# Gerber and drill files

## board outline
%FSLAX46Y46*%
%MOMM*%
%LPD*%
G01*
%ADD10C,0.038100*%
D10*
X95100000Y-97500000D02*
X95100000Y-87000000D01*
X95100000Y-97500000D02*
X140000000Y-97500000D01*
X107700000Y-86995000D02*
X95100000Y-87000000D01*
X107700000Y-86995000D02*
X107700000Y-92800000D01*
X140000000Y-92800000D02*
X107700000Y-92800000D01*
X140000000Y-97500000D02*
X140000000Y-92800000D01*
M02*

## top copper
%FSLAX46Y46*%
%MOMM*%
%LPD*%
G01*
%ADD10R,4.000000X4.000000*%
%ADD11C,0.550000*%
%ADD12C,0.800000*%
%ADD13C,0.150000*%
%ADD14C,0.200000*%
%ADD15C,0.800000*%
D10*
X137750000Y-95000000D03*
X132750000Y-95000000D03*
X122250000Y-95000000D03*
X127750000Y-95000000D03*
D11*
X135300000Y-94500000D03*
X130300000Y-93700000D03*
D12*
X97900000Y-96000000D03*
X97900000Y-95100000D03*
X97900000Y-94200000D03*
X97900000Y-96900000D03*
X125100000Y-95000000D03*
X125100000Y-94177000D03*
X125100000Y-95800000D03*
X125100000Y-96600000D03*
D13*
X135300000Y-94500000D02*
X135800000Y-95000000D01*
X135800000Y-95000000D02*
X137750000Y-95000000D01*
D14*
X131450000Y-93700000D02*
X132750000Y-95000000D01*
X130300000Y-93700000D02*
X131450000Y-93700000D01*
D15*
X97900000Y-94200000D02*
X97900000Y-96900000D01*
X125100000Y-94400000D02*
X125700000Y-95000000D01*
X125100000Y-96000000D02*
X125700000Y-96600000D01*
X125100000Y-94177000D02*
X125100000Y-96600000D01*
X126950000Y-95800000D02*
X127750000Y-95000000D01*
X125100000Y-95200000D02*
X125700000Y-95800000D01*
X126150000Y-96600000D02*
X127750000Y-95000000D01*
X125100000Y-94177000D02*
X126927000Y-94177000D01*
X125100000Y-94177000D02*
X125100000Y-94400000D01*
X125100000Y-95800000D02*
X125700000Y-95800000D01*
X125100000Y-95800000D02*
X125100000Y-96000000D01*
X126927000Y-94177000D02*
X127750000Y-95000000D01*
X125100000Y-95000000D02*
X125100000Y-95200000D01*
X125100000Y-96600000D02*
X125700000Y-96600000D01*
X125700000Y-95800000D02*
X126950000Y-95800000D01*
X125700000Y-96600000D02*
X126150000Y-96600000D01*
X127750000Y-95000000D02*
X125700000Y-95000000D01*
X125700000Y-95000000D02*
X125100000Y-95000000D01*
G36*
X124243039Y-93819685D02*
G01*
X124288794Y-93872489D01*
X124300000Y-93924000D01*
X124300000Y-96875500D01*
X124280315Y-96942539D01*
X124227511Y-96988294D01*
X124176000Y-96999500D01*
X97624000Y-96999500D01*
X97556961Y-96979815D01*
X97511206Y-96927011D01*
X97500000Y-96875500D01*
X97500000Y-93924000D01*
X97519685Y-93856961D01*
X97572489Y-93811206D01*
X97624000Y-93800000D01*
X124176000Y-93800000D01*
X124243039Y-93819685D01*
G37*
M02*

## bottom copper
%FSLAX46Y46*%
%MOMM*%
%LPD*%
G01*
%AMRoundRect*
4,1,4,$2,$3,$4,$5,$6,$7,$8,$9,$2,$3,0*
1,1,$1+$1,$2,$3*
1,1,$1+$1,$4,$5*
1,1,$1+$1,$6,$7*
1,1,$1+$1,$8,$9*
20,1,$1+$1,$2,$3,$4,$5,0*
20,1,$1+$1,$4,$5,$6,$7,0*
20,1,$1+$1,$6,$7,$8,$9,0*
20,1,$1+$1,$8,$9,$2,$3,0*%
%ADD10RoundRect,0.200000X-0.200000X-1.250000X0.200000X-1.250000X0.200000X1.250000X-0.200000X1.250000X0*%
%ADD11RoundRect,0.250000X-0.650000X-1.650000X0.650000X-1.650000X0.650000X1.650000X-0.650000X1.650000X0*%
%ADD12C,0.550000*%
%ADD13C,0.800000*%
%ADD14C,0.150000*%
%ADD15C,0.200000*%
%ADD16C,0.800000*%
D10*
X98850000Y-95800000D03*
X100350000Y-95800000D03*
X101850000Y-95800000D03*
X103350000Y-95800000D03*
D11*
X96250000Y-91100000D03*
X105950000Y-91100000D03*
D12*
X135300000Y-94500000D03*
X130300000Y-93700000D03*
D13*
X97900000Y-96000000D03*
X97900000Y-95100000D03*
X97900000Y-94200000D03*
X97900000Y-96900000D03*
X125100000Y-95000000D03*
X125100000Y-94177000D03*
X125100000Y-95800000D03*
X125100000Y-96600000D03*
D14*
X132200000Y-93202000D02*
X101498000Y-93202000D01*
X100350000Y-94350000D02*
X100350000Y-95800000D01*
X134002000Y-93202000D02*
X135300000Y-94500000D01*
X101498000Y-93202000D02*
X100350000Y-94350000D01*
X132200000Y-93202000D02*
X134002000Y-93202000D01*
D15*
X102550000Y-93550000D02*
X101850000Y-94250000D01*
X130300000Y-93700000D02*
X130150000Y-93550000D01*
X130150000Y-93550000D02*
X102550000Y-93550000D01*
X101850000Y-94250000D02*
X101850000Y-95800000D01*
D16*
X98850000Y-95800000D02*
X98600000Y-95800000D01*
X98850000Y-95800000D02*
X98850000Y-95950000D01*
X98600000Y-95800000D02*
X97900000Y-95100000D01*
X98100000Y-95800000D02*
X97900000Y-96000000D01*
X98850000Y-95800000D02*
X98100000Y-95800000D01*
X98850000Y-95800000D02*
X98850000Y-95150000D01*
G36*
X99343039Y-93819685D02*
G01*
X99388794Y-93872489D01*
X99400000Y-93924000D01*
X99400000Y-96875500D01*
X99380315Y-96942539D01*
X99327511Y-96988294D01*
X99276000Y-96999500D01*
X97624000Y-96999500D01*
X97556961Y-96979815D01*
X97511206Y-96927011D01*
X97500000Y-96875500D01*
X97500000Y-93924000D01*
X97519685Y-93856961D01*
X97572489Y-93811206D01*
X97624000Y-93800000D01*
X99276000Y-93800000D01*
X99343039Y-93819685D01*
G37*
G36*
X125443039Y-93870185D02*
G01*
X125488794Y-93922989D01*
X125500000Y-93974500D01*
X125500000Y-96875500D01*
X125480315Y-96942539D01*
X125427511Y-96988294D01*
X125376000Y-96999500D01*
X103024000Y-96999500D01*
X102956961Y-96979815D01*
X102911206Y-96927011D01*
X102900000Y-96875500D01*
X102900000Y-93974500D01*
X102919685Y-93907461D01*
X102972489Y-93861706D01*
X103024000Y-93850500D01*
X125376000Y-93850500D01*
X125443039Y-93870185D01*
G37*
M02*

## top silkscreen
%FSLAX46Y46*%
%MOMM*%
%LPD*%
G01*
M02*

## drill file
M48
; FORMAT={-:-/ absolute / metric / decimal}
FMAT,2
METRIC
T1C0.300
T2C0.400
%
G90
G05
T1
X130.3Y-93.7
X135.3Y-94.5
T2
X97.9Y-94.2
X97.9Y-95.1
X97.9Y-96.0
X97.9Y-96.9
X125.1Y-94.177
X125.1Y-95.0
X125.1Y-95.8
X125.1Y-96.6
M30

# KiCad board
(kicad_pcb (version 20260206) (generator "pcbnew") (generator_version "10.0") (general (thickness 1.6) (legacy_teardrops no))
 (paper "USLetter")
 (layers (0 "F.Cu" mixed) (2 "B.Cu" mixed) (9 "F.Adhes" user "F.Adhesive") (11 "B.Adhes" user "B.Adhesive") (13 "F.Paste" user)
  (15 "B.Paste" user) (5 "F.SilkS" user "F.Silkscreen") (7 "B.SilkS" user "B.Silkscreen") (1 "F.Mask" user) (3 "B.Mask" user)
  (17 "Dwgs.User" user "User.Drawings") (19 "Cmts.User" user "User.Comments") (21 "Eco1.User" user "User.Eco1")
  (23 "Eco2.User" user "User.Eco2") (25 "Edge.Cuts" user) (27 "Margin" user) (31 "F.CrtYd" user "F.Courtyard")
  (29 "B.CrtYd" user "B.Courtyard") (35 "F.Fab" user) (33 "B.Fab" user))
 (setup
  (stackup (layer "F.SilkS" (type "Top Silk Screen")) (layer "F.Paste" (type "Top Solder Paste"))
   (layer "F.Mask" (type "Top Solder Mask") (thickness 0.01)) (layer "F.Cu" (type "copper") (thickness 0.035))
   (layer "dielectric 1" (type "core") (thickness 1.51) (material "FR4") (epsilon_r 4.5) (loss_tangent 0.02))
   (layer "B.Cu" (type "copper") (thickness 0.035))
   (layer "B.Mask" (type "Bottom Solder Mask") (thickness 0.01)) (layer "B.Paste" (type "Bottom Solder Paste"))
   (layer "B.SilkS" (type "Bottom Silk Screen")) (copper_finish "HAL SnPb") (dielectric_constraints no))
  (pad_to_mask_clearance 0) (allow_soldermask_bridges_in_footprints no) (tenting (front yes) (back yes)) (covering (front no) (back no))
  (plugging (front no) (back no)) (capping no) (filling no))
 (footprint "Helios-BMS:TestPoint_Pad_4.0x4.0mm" (layer "F.Cu") (at 137.75 95)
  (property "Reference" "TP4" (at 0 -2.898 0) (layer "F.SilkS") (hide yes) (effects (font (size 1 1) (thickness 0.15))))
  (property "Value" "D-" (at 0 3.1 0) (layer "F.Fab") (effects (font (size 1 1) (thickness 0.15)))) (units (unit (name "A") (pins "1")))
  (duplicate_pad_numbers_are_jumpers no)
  (pad "1" smd rect (at 0 0) (size 4 4) (layers "F.Cu" "F.Mask") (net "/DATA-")))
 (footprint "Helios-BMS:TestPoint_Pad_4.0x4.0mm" (layer "F.Cu") (at 133.25 95)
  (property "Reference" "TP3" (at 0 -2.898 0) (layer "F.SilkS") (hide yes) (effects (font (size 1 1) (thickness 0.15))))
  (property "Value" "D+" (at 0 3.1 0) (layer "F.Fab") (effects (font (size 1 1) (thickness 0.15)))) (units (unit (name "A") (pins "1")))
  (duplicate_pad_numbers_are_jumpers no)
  (pad "1" smd rect (at -0.5 0) (size 4 4) (layers "F.Cu" "F.Mask") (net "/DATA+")))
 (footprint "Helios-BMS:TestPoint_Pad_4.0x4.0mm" (layer "F.Cu") (at 131 95)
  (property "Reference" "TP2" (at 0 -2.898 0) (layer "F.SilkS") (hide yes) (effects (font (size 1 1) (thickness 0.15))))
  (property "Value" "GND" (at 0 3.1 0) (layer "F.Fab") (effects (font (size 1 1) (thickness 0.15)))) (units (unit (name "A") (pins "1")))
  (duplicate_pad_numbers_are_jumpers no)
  (pad "1" smd rect (at -8.75 0) (size 4 4) (layers "F.Cu" "F.Mask") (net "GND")))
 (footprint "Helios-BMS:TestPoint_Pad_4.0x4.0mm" (layer "F.Cu") (at 122.75 95)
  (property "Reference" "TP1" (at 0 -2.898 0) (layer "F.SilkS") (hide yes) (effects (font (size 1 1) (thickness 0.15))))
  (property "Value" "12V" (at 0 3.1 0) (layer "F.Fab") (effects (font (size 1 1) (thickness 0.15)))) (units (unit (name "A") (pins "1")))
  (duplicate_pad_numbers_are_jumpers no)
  (pad "1" smd rect (at 5 0) (size 4 4) (layers "F.Cu" "F.Mask") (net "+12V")))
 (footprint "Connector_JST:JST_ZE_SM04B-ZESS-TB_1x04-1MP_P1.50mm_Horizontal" (layer "B.Cu") (at 101.1 93.225)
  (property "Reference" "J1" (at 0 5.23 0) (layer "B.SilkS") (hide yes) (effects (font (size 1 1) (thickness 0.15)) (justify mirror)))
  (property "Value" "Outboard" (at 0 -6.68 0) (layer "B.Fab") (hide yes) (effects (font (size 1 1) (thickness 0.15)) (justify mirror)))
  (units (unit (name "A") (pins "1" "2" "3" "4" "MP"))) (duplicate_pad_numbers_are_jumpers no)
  (pad "1" smd roundrect (at -2.25 2.575) (size 0.8 2.9) (layers "B.Cu" "B.Mask" "B.Paste") (roundrect_rratio 0.25) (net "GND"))
  (pad "2" smd roundrect (at -0.75 2.575) (size 0.8 2.9) (layers "B.Cu" "B.Mask" "B.Paste") (roundrect_rratio 0.25) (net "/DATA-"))
  (pad "3" smd roundrect (at 0.75 2.575) (size 0.8 2.9) (layers "B.Cu" "B.Mask" "B.Paste") (roundrect_rratio 0.25) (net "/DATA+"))
  (pad "4" smd roundrect (at 2.25 2.575) (size 0.8 2.9) (layers "B.Cu" "B.Mask" "B.Paste") (roundrect_rratio 0.25) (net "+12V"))
  (pad "MP" smd roundrect (at -4.85 -2.125) (size 1.8 3.8) (layers "B.Cu" "B.Mask" "B.Paste") (roundrect_rratio 0.138889)
   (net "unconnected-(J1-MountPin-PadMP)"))
  (pad "MP" smd roundrect (at 4.85 -2.125) (size 1.8 3.8) (layers "B.Cu" "B.Mask" "B.Paste") (roundrect_rratio 0.138889)
   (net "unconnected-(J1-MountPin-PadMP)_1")))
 (gr_line (start 95.1 97.5) (end 95.1 87) (stroke (width 0.0381) (type default)) (layer "Edge.Cuts"))
 (gr_line (start 95.1 97.5) (end 140 97.5) (stroke (width 0.0381) (type solid)) (layer "Edge.Cuts"))
 (gr_line (start 107.7 86.995) (end 95.1 87) (stroke (width 0.0381) (type default)) (layer "Edge.Cuts"))
 (gr_line (start 107.7 86.995) (end 107.7 92.8) (stroke (width 0.0381) (type default)) (layer "Edge.Cuts"))
 (gr_line (start 140 92.8) (end 107.7 92.8) (stroke (width 0.0381) (type default)) (layer "Edge.Cuts"))
 (gr_line (start 140 97.5) (end 140 92.8) (stroke (width 0.0381) (type solid)) (layer "Edge.Cuts"))
 (segment (start 135.3 94.5) (end 135.8 95) (width 0.15) (layer "F.Cu") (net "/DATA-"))
 (segment (start 135.8 95) (end 137.75 95) (width 0.15) (layer "F.Cu") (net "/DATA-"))
 (via (at 135.3 94.5) (size 0.55) (drill 0.3) (layers "F.Cu" "B.Cu") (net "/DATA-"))
 (segment (start 132.2 93.202) (end 101.498 93.202) (width 0.15) (layer "B.Cu") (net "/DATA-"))
 (segment (start 100.35 94.35) (end 100.35 95.8) (width 0.15) (layer "B.Cu") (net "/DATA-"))
 (segment (start 134.002 93.202) (end 135.3 94.5) (width 0.15) (layer "B.Cu") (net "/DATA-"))
 (segment (start 101.498 93.202) (end 100.35 94.35) (width 0.15) (layer "B.Cu") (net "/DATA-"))
 (segment (start 132.2 93.202) (end 134.002 93.202) (width 0.15) (layer "B.Cu") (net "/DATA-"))
 (segment (start 131.45 93.7) (end 132.75 95) (width 0.2) (layer "F.Cu") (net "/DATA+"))
 (segment (start 130.3 93.7) (end 131.45 93.7) (width 0.2) (layer "F.Cu") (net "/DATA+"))
 (via (at 130.3 93.7) (size 0.55) (drill 0.3) (layers "F.Cu" "B.Cu") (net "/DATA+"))
 (segment (start 102.55 93.55) (end 101.85 94.25) (width 0.2) (layer "B.Cu") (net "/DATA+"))
 (segment (start 130.3 93.7) (end 130.15 93.55) (width 0.2) (layer "B.Cu") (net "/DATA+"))
 (segment (start 130.15 93.55) (end 102.55 93.55) (width 0.2) (layer "B.Cu") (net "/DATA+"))
 (segment (start 101.85 94.25) (end 101.85 95.8) (width 0.2) (layer "B.Cu") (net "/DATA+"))
 (segment (start 97.9 94.2) (end 97.9 96.9) (width 0.8) (layer "F.Cu") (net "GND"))
 (via (at 97.9 96) (size 0.8) (drill 0.4) (layers "F.Cu" "B.Cu") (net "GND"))
 (via (at 97.9 95.1) (size 0.8) (drill 0.4) (layers "F.Cu" "B.Cu") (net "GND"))
 (via (at 97.9 94.2) (size 0.8) (drill 0.4) (layers "F.Cu" "B.Cu") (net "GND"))
 (via (at 97.9 96.9) (size 0.8) (drill 0.4) (layers "F.Cu" "B.Cu") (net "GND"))
 (segment (start 98.85 95.8) (end 98.6 95.8) (width 0.8) (layer "B.Cu") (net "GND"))
 (segment (start 98.85 95.8) (end 98.85 95.95) (width 0.8) (layer "B.Cu") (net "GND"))
 (segment (start 98.6 95.8) (end 97.9 95.1) (width 0.8) (layer "B.Cu") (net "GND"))
 (segment (start 98.1 95.8) (end 97.9 96) (width 0.8) (layer "B.Cu") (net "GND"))
 (segment (start 98.85 95.8) (end 98.1 95.8) (width 0.8) (layer "B.Cu") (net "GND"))
 (segment (start 98.85 95.8) (end 98.85 95.15) (width 0.8) (layer "B.Cu") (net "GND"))
 (segment (start 125.1 94.4) (end 125.7 95) (width 0.8) (layer "F.Cu") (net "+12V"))
 (segment (start 125.1 96) (end 125.7 96.6) (width 0.8) (layer "F.Cu") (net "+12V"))
 (segment (start 125.1 94.177) (end 125.1 96.6) (width 0.8) (layer "F.Cu") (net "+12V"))
 (segment (start 126.95 95.8) (end 127.75 95) (width 0.8) (layer "F.Cu") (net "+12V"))
 (segment (start 125.1 95.2) (end 125.7 95.8) (width 0.8) (layer "F.Cu") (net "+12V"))
 (segment (start 126.15 96.6) (end 127.75 95) (width 0.8) (layer "F.Cu") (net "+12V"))
 (segment (start 125.1 94.177) (end 126.927 94.177) (width 0.8) (layer "F.Cu") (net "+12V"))
 (segment (start 125.1 94.177) (end 125.1 94.4) (width 0.8) (layer "F.Cu") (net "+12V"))
 (segment (start 125.1 95.8) (end 125.7 95.8) (width 0.8) (layer "F.Cu") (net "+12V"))
 (segment (start 125.1 95.8) (end 125.1 96) (width 0.8) (layer "F.Cu") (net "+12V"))
 (segment (start 126.927 94.177) (end 127.75 95) (width 0.8) (layer "F.Cu") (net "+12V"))
 (segment (start 125.1 95) (end 125.1 95.2) (width 0.8) (layer "F.Cu") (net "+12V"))
 (segment (start 125.1 96.6) (end 125.7 96.6) (width 0.8) (layer "F.Cu") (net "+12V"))
 (segment (start 125.7 95.8) (end 126.95 95.8) (width 0.8) (layer "F.Cu") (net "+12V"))
 (segment (start 125.7 96.6) (end 126.15 96.6) (width 0.8) (layer "F.Cu") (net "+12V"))
 (segment (start 127.75 95) (end 125.7 95) (width 0.8) (layer "F.Cu") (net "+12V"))
 (segment (start 125.7 95) (end 125.1 95) (width 0.8) (layer "F.Cu") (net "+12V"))
 (via (at 125.1 95) (size 0.8) (drill 0.4) (layers "F.Cu" "B.Cu") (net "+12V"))
 (via (at 125.1 94.177) (size 0.8) (drill 0.4) (layers "F.Cu" "B.Cu") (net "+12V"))
 (via (at 125.1 95.8) (size 0.8) (drill 0.4) (layers "F.Cu" "B.Cu") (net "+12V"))
 (via (at 125.1 96.6) (size 0.8) (drill 0.4) (layers "F.Cu" "B.Cu") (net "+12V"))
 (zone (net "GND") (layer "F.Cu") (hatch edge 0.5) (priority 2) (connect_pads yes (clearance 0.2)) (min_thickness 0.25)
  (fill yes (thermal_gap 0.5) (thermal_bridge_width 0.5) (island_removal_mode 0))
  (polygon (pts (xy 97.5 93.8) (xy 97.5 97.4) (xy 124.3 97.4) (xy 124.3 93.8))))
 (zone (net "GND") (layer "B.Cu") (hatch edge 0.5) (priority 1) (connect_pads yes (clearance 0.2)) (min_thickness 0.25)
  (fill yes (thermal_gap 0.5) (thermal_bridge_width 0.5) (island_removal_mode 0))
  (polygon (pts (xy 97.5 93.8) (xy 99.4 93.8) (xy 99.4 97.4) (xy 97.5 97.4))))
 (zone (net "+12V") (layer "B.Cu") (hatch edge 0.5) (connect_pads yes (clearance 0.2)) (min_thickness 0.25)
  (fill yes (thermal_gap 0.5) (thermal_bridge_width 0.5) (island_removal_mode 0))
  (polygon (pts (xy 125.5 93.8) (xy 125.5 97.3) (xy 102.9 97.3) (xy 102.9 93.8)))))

